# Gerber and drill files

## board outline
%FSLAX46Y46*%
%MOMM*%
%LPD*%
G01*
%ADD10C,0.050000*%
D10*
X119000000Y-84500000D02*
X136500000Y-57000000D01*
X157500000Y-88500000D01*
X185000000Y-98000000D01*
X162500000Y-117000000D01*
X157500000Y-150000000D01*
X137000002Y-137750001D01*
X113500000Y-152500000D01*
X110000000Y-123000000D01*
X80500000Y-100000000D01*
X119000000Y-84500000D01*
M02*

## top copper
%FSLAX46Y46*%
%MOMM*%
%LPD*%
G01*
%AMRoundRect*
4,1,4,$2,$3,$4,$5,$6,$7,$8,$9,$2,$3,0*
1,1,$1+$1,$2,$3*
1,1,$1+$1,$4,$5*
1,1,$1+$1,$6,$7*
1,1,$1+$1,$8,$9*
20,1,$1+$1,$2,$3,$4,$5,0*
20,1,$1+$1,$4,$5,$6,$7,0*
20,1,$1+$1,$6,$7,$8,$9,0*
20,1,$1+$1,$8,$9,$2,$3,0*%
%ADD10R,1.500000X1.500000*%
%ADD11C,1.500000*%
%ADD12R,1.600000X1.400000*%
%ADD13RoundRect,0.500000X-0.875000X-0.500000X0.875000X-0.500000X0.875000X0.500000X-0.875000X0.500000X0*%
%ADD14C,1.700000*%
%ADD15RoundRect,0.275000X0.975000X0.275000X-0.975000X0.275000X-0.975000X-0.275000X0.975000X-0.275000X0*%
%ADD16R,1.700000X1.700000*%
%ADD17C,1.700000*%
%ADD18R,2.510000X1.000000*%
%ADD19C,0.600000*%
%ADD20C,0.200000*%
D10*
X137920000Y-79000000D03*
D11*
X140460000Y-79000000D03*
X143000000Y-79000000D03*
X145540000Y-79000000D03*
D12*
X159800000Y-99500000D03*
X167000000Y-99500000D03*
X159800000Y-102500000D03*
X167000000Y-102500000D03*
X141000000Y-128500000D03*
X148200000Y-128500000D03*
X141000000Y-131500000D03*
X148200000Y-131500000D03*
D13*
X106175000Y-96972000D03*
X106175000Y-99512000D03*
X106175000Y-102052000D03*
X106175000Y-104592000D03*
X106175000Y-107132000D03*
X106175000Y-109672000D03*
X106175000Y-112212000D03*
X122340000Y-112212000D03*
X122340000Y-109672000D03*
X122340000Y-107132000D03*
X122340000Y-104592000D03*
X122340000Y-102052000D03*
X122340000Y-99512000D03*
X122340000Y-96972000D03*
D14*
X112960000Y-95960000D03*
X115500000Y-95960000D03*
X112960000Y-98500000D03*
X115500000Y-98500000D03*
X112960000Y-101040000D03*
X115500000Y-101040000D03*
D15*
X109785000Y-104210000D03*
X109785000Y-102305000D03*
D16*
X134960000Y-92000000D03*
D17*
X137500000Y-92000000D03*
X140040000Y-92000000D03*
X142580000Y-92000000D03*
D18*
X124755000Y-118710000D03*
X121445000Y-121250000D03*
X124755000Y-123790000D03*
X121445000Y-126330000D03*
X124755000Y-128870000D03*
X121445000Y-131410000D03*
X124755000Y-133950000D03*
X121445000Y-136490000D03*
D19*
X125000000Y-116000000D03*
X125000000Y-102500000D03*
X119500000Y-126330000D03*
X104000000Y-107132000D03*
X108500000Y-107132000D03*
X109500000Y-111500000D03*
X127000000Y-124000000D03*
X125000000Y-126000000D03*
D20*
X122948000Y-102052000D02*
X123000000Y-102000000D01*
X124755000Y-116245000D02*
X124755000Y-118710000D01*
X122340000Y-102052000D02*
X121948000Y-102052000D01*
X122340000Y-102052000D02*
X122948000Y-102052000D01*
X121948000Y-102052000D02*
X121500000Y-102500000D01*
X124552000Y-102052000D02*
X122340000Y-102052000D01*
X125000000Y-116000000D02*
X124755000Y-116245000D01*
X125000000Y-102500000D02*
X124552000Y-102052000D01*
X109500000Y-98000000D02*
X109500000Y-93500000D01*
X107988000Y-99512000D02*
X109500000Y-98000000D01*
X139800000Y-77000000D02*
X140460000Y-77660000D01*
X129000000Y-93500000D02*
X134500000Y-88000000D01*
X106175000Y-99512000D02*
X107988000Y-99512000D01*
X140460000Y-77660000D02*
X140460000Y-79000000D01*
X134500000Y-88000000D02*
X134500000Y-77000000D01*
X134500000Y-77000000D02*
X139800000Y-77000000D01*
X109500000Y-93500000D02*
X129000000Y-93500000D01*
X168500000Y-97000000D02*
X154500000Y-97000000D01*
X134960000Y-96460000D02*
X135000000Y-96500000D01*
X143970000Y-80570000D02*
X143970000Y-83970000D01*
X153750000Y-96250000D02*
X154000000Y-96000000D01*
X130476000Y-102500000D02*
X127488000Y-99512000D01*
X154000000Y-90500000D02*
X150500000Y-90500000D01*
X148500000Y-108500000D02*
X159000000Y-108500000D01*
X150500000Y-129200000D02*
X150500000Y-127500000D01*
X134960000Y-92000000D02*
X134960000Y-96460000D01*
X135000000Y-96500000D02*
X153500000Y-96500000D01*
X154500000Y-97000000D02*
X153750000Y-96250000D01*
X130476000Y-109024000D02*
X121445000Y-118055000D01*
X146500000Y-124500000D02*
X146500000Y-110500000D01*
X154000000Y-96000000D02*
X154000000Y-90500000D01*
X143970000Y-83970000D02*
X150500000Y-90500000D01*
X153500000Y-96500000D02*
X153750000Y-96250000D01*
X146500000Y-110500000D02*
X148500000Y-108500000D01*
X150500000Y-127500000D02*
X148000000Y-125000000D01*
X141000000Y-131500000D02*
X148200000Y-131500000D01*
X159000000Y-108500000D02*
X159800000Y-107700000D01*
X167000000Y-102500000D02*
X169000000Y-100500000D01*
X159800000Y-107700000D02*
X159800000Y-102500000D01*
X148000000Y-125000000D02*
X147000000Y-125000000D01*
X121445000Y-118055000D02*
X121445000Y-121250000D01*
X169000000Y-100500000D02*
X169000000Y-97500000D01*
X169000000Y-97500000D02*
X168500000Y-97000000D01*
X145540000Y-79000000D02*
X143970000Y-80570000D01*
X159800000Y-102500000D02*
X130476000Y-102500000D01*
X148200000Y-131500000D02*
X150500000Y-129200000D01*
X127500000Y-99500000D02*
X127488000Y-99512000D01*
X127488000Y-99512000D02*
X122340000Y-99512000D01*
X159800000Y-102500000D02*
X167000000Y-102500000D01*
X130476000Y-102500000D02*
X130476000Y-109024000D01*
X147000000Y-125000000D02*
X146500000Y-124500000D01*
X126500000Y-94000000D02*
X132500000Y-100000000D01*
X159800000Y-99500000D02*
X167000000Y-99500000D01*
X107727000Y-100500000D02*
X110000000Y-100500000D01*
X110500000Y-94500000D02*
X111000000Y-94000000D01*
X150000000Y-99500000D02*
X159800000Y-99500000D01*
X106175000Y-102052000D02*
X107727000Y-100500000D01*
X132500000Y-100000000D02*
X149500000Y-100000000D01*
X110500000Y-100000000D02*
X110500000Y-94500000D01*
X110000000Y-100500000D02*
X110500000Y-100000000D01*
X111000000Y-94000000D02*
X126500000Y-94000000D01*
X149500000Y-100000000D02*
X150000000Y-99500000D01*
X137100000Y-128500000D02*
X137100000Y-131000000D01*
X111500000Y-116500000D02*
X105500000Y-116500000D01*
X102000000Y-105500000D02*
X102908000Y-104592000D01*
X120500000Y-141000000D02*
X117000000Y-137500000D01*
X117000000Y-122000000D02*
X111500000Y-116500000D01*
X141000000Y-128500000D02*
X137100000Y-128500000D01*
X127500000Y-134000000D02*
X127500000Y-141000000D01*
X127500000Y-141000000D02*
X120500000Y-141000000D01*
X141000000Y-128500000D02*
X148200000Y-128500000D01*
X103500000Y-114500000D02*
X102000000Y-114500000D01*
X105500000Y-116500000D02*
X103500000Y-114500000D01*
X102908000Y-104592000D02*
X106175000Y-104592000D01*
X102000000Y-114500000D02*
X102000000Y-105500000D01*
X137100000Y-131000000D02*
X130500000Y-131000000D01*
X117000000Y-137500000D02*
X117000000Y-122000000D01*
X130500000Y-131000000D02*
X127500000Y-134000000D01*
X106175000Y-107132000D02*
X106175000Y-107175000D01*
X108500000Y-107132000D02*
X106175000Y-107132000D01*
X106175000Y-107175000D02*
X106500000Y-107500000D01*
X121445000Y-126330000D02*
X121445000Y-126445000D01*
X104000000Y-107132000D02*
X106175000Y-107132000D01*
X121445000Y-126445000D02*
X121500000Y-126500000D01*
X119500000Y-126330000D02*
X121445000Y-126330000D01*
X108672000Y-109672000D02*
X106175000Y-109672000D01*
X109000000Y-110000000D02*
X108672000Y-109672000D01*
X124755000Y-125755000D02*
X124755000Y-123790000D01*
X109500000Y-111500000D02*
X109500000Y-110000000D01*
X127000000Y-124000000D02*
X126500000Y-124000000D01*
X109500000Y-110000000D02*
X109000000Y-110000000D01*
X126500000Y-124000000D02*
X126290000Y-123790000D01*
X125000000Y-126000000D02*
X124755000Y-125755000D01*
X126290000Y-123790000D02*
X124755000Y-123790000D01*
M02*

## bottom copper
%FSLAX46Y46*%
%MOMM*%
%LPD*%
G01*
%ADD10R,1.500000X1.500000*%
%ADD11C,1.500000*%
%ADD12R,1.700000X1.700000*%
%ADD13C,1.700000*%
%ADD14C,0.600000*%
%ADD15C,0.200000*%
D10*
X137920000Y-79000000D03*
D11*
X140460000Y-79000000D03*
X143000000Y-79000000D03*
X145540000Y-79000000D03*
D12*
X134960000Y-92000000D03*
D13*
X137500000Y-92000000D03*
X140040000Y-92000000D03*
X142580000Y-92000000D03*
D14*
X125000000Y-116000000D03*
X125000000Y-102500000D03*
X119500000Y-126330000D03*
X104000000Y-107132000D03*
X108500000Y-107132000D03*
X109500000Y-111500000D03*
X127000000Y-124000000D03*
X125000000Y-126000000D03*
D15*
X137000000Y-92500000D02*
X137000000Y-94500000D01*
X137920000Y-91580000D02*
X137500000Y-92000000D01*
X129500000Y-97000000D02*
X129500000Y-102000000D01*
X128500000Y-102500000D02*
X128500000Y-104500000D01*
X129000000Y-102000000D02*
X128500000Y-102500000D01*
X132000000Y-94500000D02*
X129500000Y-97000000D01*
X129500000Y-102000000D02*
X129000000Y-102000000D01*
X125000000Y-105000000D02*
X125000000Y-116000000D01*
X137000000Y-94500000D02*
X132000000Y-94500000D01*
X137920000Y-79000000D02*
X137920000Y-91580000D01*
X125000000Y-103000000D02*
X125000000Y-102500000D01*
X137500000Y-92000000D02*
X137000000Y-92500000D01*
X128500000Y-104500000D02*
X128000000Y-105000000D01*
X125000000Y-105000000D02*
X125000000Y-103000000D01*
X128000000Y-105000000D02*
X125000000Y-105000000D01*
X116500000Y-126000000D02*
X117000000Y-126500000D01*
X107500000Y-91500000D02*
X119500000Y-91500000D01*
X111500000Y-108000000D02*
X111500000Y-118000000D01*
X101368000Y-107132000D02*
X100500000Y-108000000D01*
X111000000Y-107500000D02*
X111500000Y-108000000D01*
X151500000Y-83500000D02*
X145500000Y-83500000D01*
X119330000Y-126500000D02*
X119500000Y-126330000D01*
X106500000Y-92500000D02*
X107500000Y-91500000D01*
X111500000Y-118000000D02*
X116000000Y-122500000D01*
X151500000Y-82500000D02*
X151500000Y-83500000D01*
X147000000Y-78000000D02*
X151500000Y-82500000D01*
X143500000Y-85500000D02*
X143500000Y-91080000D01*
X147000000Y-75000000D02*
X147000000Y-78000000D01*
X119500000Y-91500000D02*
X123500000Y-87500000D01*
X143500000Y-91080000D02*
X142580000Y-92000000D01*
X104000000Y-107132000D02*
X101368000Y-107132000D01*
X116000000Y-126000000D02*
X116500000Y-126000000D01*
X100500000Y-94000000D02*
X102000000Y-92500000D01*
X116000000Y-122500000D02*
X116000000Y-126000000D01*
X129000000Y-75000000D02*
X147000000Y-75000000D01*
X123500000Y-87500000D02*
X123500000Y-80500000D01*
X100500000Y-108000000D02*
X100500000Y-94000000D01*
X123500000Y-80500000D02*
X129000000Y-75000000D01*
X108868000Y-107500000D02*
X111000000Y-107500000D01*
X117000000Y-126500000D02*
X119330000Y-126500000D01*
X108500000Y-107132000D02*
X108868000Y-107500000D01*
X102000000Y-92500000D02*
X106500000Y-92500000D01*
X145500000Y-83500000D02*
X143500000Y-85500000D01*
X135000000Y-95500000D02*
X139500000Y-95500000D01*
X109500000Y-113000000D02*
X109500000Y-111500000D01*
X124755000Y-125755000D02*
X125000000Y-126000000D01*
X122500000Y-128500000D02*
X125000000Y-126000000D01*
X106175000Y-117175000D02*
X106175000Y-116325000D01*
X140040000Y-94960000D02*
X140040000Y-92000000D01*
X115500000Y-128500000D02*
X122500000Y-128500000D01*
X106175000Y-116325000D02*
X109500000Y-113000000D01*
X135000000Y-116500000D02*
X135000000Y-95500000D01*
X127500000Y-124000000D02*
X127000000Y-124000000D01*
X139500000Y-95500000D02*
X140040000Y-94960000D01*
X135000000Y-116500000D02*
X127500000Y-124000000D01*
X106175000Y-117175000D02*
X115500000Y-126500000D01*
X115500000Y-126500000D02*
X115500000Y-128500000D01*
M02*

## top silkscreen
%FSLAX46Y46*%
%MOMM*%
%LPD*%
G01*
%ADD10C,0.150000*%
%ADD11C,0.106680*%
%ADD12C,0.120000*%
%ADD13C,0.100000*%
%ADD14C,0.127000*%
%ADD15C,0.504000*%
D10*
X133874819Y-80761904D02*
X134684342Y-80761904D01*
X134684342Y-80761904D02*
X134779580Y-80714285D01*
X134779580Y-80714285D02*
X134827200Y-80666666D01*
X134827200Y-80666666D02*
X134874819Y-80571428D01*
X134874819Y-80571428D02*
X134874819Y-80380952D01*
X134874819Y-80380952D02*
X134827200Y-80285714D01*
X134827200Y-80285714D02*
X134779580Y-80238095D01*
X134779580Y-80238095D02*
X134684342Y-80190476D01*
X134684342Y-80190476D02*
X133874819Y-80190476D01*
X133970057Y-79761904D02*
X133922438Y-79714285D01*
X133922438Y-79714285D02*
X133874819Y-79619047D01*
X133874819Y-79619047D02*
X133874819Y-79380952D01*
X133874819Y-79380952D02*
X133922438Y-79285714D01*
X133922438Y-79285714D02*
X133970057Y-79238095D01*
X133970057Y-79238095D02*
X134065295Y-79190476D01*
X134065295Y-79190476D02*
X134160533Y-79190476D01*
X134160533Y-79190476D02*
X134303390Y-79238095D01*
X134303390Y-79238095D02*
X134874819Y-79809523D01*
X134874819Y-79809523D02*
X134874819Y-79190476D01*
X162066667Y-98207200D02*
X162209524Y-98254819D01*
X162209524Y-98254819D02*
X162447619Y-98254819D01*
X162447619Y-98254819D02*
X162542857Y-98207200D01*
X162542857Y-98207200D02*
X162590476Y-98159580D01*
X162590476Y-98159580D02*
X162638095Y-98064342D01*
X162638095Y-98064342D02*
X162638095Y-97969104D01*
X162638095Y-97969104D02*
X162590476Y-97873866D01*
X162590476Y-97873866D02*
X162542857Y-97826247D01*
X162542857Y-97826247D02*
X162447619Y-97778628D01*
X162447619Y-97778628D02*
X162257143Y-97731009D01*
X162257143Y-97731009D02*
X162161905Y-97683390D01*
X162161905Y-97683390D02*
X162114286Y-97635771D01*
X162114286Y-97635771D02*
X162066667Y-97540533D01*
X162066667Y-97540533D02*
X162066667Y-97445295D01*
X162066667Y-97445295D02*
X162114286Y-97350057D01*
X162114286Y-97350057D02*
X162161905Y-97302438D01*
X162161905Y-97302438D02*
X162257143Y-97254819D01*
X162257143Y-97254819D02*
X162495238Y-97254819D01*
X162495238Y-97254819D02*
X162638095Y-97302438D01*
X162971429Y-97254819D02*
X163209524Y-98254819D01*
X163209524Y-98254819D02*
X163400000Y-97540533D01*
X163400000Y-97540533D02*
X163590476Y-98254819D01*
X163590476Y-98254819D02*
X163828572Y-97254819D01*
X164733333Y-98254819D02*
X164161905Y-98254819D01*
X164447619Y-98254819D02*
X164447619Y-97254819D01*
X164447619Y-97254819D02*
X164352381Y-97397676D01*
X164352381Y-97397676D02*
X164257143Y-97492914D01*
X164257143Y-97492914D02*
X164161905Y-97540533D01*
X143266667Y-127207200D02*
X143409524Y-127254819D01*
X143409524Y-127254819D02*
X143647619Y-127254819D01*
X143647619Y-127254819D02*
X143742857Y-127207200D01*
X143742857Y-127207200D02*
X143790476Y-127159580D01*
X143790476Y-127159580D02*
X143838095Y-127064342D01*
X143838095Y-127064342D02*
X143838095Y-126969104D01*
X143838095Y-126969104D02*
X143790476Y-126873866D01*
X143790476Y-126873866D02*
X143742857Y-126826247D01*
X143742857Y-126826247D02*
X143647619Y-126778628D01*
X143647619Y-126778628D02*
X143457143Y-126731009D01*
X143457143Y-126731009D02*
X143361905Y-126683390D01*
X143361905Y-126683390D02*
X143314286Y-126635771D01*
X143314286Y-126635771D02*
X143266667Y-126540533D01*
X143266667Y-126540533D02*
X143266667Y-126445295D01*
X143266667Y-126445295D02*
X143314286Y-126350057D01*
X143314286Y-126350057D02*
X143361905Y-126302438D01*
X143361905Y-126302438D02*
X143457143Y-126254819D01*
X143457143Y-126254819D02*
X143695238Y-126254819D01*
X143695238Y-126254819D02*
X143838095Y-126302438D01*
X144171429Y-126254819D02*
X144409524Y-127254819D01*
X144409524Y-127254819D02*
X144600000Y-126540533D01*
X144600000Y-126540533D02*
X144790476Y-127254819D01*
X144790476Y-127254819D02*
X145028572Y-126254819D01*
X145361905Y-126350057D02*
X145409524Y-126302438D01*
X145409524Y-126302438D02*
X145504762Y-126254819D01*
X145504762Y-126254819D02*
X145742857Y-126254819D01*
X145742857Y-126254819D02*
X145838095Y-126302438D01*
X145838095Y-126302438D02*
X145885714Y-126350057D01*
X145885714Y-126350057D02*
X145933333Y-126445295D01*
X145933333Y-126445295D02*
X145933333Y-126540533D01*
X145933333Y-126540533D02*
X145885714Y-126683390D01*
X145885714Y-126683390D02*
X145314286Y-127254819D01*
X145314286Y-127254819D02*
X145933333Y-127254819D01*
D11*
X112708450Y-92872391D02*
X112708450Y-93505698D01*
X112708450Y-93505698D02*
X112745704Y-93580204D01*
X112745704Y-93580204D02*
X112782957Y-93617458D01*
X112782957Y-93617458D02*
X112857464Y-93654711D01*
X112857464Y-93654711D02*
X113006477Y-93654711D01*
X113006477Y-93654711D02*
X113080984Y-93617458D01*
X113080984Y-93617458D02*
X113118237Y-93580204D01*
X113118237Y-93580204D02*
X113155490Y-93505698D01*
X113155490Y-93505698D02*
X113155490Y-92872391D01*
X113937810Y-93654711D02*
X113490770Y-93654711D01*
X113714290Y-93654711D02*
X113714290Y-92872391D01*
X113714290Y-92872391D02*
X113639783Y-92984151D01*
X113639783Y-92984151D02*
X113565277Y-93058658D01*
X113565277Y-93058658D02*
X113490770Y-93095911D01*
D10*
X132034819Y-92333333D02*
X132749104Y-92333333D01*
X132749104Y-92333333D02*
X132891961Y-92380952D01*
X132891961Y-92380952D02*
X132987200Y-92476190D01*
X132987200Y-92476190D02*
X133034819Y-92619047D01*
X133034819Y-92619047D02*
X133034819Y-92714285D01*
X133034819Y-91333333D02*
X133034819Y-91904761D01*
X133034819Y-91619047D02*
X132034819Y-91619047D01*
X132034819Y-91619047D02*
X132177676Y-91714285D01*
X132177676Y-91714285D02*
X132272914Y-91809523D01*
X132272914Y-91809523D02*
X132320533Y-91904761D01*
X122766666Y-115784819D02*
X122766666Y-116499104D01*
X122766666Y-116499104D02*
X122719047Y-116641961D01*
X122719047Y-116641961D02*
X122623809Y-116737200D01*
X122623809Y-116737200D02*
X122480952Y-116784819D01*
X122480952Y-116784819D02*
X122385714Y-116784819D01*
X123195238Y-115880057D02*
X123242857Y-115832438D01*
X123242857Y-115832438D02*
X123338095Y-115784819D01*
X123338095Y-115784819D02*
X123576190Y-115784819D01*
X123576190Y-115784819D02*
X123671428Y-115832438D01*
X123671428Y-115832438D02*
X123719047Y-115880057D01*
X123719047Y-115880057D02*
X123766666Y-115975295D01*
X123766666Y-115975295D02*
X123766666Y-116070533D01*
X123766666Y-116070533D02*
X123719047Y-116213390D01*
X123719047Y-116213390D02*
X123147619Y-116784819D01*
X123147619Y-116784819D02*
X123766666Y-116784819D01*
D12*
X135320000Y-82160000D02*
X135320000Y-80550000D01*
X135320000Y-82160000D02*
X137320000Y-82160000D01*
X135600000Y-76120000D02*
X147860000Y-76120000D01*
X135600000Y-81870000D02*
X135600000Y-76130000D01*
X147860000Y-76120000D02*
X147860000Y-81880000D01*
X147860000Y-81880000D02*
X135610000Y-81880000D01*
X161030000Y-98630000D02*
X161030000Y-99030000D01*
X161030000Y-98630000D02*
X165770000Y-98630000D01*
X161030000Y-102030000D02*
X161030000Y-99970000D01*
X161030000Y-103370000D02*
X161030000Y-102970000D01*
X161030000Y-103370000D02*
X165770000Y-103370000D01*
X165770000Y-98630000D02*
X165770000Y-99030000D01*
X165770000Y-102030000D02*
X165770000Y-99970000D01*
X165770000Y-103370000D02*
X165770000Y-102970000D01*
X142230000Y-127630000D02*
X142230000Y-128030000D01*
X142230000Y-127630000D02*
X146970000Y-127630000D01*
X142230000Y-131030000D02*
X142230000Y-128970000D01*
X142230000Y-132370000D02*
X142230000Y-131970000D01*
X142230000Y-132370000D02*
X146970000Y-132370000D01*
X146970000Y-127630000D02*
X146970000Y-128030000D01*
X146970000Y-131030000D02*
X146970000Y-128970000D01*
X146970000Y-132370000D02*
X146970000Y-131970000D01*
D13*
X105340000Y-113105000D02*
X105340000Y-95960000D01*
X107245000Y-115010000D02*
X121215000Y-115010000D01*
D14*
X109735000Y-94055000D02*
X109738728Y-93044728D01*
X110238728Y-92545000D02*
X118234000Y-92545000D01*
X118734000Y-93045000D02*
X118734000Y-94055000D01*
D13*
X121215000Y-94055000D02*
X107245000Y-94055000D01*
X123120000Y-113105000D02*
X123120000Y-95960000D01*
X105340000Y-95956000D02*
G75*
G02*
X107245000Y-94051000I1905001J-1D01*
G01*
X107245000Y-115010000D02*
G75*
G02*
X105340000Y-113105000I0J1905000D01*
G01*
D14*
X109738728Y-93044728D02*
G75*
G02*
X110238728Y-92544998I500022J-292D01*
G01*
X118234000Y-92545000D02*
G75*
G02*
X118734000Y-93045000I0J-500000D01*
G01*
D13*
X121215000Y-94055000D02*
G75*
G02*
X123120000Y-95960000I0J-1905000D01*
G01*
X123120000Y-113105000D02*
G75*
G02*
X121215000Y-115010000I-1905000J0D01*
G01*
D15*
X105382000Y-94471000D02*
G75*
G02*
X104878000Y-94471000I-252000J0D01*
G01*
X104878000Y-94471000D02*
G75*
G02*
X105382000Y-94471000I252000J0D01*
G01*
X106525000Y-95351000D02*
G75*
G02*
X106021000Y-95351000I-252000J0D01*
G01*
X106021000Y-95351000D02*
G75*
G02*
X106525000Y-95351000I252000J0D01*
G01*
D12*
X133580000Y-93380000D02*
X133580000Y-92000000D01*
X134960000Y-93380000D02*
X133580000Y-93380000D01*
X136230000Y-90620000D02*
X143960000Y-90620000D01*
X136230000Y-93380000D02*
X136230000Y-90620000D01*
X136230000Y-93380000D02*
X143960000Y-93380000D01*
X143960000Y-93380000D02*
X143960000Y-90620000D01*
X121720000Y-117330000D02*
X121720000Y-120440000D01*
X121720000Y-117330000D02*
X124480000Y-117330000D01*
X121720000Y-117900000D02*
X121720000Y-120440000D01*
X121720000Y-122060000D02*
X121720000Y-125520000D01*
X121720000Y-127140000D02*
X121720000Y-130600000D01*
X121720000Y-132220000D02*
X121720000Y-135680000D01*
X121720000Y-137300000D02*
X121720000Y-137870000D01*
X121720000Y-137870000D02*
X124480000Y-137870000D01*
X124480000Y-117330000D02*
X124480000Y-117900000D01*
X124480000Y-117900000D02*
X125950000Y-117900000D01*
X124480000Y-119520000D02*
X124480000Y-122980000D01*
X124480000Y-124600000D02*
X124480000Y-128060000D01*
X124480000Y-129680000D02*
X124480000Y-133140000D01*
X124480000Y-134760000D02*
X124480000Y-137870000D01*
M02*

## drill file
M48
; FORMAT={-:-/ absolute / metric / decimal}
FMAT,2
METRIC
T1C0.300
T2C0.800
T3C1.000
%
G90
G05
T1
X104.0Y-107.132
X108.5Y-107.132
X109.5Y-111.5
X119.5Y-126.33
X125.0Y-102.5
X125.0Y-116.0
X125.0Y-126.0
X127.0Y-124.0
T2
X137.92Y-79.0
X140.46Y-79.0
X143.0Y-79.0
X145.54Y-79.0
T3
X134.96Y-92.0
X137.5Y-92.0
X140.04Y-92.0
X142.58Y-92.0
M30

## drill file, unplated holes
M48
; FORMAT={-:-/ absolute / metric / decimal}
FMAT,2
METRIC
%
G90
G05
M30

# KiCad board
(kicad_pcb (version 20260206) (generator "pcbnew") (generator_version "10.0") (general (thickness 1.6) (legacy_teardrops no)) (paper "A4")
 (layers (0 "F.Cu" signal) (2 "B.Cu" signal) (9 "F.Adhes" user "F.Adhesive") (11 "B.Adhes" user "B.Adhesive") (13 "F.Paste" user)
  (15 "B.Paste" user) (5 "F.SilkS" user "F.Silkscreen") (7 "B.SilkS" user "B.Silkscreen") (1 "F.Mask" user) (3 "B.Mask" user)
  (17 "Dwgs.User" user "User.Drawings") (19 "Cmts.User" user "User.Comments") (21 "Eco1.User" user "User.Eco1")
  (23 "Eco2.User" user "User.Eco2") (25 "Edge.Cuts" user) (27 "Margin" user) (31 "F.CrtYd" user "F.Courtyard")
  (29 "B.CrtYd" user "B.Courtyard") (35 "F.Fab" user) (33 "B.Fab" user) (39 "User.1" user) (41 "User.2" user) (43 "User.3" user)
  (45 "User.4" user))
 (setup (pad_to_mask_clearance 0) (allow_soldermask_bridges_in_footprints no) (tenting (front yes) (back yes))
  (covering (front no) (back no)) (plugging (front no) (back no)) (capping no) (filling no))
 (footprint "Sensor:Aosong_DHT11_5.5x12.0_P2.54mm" (layer "F.Cu") (at 137.92 79 90)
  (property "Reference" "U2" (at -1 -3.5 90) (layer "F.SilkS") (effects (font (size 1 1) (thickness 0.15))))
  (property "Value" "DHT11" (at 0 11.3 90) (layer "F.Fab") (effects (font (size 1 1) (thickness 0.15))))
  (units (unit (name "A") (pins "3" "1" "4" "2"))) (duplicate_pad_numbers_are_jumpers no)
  (fp_line (start -3.16 -2.6) (end -1.55 -2.6) (stroke (width 0.12) (type solid)) (layer "F.SilkS"))
  (fp_line (start -3.16 -2.6) (end -3.16 -0.6) (stroke (width 0.12) (type solid)) (layer "F.SilkS"))
  (fp_line (start 2.88 -2.32) (end 2.88 9.94) (stroke (width 0.12) (type solid)) (layer "F.SilkS"))
  (fp_line (start -2.87 -2.32) (end 2.87 -2.32) (stroke (width 0.12) (type solid)) (layer "F.SilkS"))
  (fp_line (start 2.88 9.94) (end -2.88 9.94) (stroke (width 0.12) (type solid)) (layer "F.SilkS"))
  (fp_line (start -2.88 9.94) (end -2.88 -2.31) (stroke (width 0.12) (type solid)) (layer "F.SilkS"))
  (pad "1" thru_hole rect (at 0 0 90) (size 1.5 1.5) (drill 0.8) (layers "*.Cu" "*.Mask") (remove_unused_layers no) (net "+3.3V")
   (padstack (mode custom) (layer "B.Cu" (shape rect) (size 1.5 1.5))))
  (pad "2" thru_hole circle (at 0 2.54 90) (size 1.5 1.5) (drill 0.8) (layers "*.Cu" "*.Mask") (remove_unused_layers no) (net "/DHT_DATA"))
  (pad "3" thru_hole circle (at 0 5.08 90) (size 1.5 1.5) (drill 0.8) (layers "*.Cu" "*.Mask") (remove_unused_layers no)
   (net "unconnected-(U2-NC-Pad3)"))
  (pad "4" thru_hole circle (at 0 7.62 90) (size 1.5 1.5) (drill 0.8) (layers "*.Cu" "*.Mask") (remove_unused_layers no) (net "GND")))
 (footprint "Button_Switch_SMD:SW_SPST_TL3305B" (layer "F.Cu") (at 163.4 101)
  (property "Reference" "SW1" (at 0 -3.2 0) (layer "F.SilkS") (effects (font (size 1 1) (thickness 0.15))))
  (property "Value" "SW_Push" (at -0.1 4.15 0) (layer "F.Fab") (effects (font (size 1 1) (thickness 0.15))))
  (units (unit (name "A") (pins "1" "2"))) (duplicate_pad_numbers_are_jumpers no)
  (fp_line (start -2.37 -2.37) (end -2.37 -1.97) (stroke (width 0.12) (type solid)) (layer "F.SilkS"))
  (fp_line (start -2.37 -2.37) (end 2.37 -2.37) (stroke (width 0.12) (type solid)) (layer "F.SilkS"))
  (fp_line (start -2.37 1.03) (end -2.37 -1.03) (stroke (width 0.12) (type solid)) (layer "F.SilkS"))
  (fp_line (start -2.37 2.37) (end -2.37 1.97) (stroke (width 0.12) (type solid)) (layer "F.SilkS"))
  (fp_line (start -2.37 2.37) (end 2.37 2.37) (stroke (width 0.12) (type solid)) (layer "F.SilkS"))
  (fp_line (start 2.37 -2.37) (end 2.37 -1.97) (stroke (width 0.12) (type solid)) (layer "F.SilkS"))
  (fp_line (start 2.37 1.03) (end 2.37 -1.03) (stroke (width 0.12) (type solid)) (layer "F.SilkS"))
  (fp_line (start 2.37 2.37) (end 2.37 1.97) (stroke (width 0.12) (type solid)) (layer "F.SilkS"))
  (pad "1" smd rect (at -3.6 -1.5) (size 1.6 1.4) (layers "F.Cu" "F.Mask" "F.Paste") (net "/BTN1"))
  (pad "1" smd rect (at 3.6 -1.5) (size 1.6 1.4) (layers "F.Cu" "F.Mask" "F.Paste") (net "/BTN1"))
  (pad "2" smd rect (at -3.6 1.5) (size 1.6 1.4) (layers "F.Cu" "F.Mask" "F.Paste") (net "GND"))
  (pad "2" smd rect (at 3.6 1.5) (size 1.6 1.4) (layers "F.Cu" "F.Mask" "F.Paste") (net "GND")))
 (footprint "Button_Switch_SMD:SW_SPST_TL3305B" (layer "F.Cu") (at 144.6 130)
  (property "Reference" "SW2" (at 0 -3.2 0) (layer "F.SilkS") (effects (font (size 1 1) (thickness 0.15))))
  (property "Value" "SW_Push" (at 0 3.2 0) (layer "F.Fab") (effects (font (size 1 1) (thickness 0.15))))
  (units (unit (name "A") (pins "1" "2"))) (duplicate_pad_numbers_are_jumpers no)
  (fp_line (start -2.37 -2.37) (end -2.37 -1.97) (stroke (width 0.12) (type solid)) (layer "F.SilkS"))
  (fp_line (start -2.37 -2.37) (end 2.37 -2.37) (stroke (width 0.12) (type solid)) (layer "F.SilkS"))
  (fp_line (start -2.37 1.03) (end -2.37 -1.03) (stroke (width 0.12) (type solid)) (layer "F.SilkS"))
  (fp_line (start -2.37 2.37) (end -2.37 1.97) (stroke (width 0.12) (type solid)) (layer "F.SilkS"))
  (fp_line (start -2.37 2.37) (end 2.37 2.37) (stroke (width 0.12) (type solid)) (layer "F.SilkS"))
  (fp_line (start 2.37 -2.37) (end 2.37 -1.97) (stroke (width 0.12) (type solid)) (layer "F.SilkS"))
  (fp_line (start 2.37 1.03) (end 2.37 -1.03) (stroke (width 0.12) (type solid)) (layer "F.SilkS"))
  (fp_line (start 2.37 2.37) (end 2.37 1.97) (stroke (width 0.12) (type solid)) (layer "F.SilkS"))
  (pad "1" smd rect (at -3.6 -1.5) (size 1.6 1.4) (layers "F.Cu" "F.Mask" "F.Paste") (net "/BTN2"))
  (pad "1" smd rect (at 3.6 -1.5) (size 1.6 1.4) (layers "F.Cu" "F.Mask" "F.Paste") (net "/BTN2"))
  (pad "2" smd rect (at -3.6 1.5) (size 1.6 1.4) (layers "F.Cu" "F.Mask" "F.Paste") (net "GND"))
  (pad "2" smd rect (at 3.6 1.5) (size 1.6 1.4) (layers "F.Cu" "F.Mask" "F.Paste") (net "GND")))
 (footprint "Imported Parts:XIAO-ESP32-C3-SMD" (layer "F.Cu") (at 105.34 115.092)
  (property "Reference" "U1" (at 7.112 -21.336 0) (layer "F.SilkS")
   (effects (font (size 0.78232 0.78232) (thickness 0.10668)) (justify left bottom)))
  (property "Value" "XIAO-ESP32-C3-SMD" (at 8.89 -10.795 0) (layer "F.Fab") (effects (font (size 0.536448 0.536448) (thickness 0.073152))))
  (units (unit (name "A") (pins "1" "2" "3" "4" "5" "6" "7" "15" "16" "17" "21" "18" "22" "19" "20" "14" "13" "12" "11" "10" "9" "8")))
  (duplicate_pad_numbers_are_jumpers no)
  (fp_line (start 0 -1.987) (end 0 -19.132) (stroke (width 0.1) (type solid)) (layer "F.SilkS"))
  (fp_line (start 1.905 -0.082) (end 15.875 -0.082) (stroke (width 0.1) (type solid)) (layer "F.SilkS"))
  (fp_line (start 4.395 -21.037) (end 4.398728 -22.047272) (stroke (width 0.127) (type solid)) (layer "F.SilkS"))
  (fp_line (start 4.898728 -22.547) (end 12.894 -22.547) (stroke (width 0.127) (type solid)) (layer "F.SilkS"))
  (fp_line (start 13.394 -22.047) (end 13.394 -21.037) (stroke (width 0.127) (type solid)) (layer "F.SilkS"))
  (fp_line (start 15.875 -21.037) (end 1.905 -21.037) (stroke (width 0.1) (type solid)) (layer "F.SilkS"))
  (fp_line (start 17.78 -1.987) (end 17.78 -19.132) (stroke (width 0.1) (type solid)) (layer "F.SilkS"))
  (fp_arc (start 0 -19.136) (mid 0.557962 -20.483038) (end 1.905 -21.041) (stroke (width 0.1) (type solid)) (layer "F.SilkS"))
  (fp_arc (start 1.905 -0.082) (mid 0.557962 -0.639962) (end 0 -1.987) (stroke (width 0.1) (type solid)) (layer "F.SilkS"))
  (fp_arc (start 4.398728 -22.047272) (mid 4.545272 -22.40064) (end 4.898728 -22.547) (stroke (width 0.127) (type default))
   (layer "F.SilkS"))
  (fp_arc (start 12.894 -22.547) (mid 13.247553 -22.400553) (end 13.394 -22.047) (stroke (width 0.127) (type default)) (layer "F.SilkS"))
  (fp_arc (start 15.875 -21.037) (mid 17.222038 -20.479038) (end 17.78 -19.132) (stroke (width 0.1) (type solid)) (layer "F.SilkS"))
  (fp_arc (start 17.78 -1.987) (mid 17.222038 -0.639962) (end 15.875 -0.082) (stroke (width 0.1) (type solid)) (layer "F.SilkS"))
  (fp_circle (center -0.21 -20.621) (end -0.21 -20.875) (stroke (width 0.5) (type solid)) (fill yes) (layer "F.SilkS"))
  (fp_circle (center 0.933 -19.741) (end 0.933 -19.995) (stroke (width 0.5) (type solid)) (fill yes) (layer "F.SilkS"))
  (pad "1" smd roundrect (at 0.835 -18.12) (size 2.75 2) (layers "F.Cu" "F.Mask" "F.Paste") (roundrect_rratio 0.25)
   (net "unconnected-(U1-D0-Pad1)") (solder_mask_margin 0.0508) (thermal_bridge_angle 45))
  (pad "2" smd roundrect (at 0.835 -15.58) (size 2.75 2) (layers "F.Cu" "F.Mask" "F.Paste") (roundrect_rratio 0.25) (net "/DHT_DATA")
   (solder_mask_margin 0.0508) (thermal_bridge_angle 45))
  (pad "3" smd roundrect (at 0.835 -13.04) (size 2.75 2) (layers "F.Cu" "F.Mask" "F.Paste") (roundrect_rratio 0.25) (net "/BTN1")
   (solder_mask_margin 0.0508) (thermal_bridge_angle 45))
  (pad "4" smd roundrect (at 0.835 -10.5) (size 2.75 2) (layers "F.Cu" "F.Mask" "F.Paste") (roundrect_rratio 0.25) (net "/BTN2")
   (solder_mask_margin 0.0508) (thermal_bridge_angle 45))
  (pad "5" smd roundrect (at 0.835 -7.96) (size 2.75 2) (layers "F.Cu" "F.Mask" "F.Paste") (roundrect_rratio 0.25) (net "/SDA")
   (solder_mask_margin 0.0508) (thermal_bridge_angle 45)
   (padstack (mode custom) (layer "B.Cu" (shape roundrect) (size 2.75 2) (roundrect_rratio 0.25))))
  (pad "6" smd roundrect (at 0.835 -5.42) (size 2.75 2) (layers "F.Cu" "F.Mask" "F.Paste") (roundrect_rratio 0.25) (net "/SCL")
   (solder_mask_margin 0.0508) (thermal_bridge_angle 45))
  (pad "7" smd roundrect (at 0.835 -2.88) (size 2.75 2) (layers "F.Cu" "F.Mask" "F.Paste") (roundrect_rratio 0.25)
   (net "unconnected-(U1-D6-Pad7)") (solder_mask_margin 0.0508) (thermal_bridge_angle 45))
  (pad "8" smd roundrect (at 17 -2.88) (size 2.75 2) (layers "F.Cu" "F.Mask" "F.Paste") (roundrect_rratio 0.25)
   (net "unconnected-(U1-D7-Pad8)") (solder_mask_margin 0.0508) (thermal_bridge_angle 45))
  (pad "9" smd roundrect (at 17 -5.42) (size 2.75 2) (layers "F.Cu" "F.Mask" "F.Paste") (roundrect_rratio 0.25)
   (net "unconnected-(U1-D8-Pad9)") (solder_mask_margin 0.0508) (thermal_bridge_angle 45))
  (pad "10" smd roundrect (at 17 -7.96) (size 2.75 2) (layers "F.Cu" "F.Mask" "F.Paste") (roundrect_rratio 0.25)
   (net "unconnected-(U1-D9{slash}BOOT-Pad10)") (solder_mask_margin 0.0508) (thermal_bridge_angle 45))
  (pad "11" smd roundrect (at 17 -10.5) (size 2.75 2) (layers "F.Cu" "F.Mask" "F.Paste") (roundrect_rratio 0.25)
   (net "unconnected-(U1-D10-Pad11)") (solder_mask_margin 0.0508) (thermal_bridge_angle 45))
  (pad "12" smd roundrect (at 17 -13.04) (size 2.75 2) (layers "F.Cu" "F.Mask" "F.Paste") (roundrect_rratio 0.25) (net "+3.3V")
   (solder_mask_margin 0.0508) (thermal_bridge_angle 45)
   (padstack (mode custom) (layer "B.Cu" (shape roundrect) (size 2.75 2) (roundrect_rratio 0.25))))
  (pad "13" smd roundrect (at 17 -15.58) (size 2.75 2) (layers "F.Cu" "F.Mask" "F.Paste") (roundrect_rratio 0.25) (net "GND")
   (solder_mask_margin 0.0508) (thermal_bridge_angle 45))
  (pad "14" smd roundrect (at 17 -18.12) (size 2.75 2) (layers "F.Cu" "F.Mask" "F.Paste") (roundrect_rratio 0.25) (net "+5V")
   (solder_mask_margin 0.0508) (thermal_bridge_angle 45))
  (pad "15" smd circle (at 7.62 -19.132) (size 1.7 1.7) (layers "F.Cu" "F.Mask" "F.Paste") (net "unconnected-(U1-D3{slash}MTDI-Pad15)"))
  (pad "16" smd circle (at 10.16 -19.132) (size 1.7 1.7) (layers "F.Cu" "F.Mask" "F.Paste") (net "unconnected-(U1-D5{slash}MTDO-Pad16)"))
  (pad "17" smd circle (at 7.62 -16.592) (size 1.7 1.7) (layers "F.Cu" "F.Mask" "F.Paste") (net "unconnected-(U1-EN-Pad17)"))
  (pad "18" smd circle (at 10.16 -16.592) (size 1.7 1.7) (layers "F.Cu" "F.Mask" "F.Paste") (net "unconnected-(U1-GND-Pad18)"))
  (pad "19" smd circle (at 7.62 -14.052) (size 1.7 1.7) (layers "F.Cu" "F.Mask" "F.Paste") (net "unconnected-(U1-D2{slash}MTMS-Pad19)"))
  (pad "20" smd circle (at 10.16 -14.052) (size 1.7 1.7) (layers "F.Cu" "F.Mask" "F.Paste") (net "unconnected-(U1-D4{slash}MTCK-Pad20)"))
  (pad "21" smd roundrect (at 4.445 -10.882 180) (size 2.5 1.1) (layers "F.Cu" "F.Mask" "F.Paste") (roundrect_rratio 0.25)
   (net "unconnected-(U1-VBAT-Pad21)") (thermal_bridge_angle 45))
  (pad "22" smd roundrect (at 4.445 -12.787 180) (size 2.5 1.1) (layers "F.Cu" "F.Mask" "F.Paste") (roundrect_rratio 0.25)
   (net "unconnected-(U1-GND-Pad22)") (thermal_bridge_angle 45)))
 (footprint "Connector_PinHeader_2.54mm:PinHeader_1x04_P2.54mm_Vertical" (layer "F.Cu") (at 134.96 92 90)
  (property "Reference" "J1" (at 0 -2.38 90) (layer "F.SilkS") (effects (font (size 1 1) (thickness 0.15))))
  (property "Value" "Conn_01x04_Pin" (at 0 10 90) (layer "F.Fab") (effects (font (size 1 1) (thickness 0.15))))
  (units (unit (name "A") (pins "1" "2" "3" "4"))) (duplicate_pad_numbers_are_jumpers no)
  (fp_line (start -1.38 -1.38) (end 0 -1.38) (stroke (width 0.12) (type solid)) (layer "F.SilkS"))
  (fp_line (start -1.38 0) (end -1.38 -1.38) (stroke (width 0.12) (type solid)) (layer "F.SilkS"))
  (fp_line (start 1.38 1.27) (end 1.38 9) (stroke (width 0.12) (type solid)) (layer "F.SilkS"))
  (fp_line (start -1.38 1.27) (end 1.38 1.27) (stroke (width 0.12) (type solid)) (layer "F.SilkS"))
  (fp_line (start -1.38 1.27) (end -1.38 9) (stroke (width 0.12) (type solid)) (layer "F.SilkS"))
  (fp_line (start -1.38 9) (end 1.38 9) (stroke (width 0.12) (type solid)) (layer "F.SilkS"))
  (pad "1" thru_hole rect (at 0 0 90) (size 1.7 1.7) (drill 1) (layers "*.Cu" "*.Mask") (remove_unused_layers no) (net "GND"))
  (pad "2" thru_hole circle (at 0 2.54 90) (size 1.7 1.7) (drill 1) (layers "*.Cu" "*.Mask") (remove_unused_layers no) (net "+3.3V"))
  (pad "3" thru_hole circle (at 0 5.08 90) (size 1.7 1.7) (drill 1) (layers "*.Cu" "*.Mask") (remove_unused_layers no) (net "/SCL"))
  (pad "4" thru_hole circle (at 0 7.62 90) (size 1.7 1.7) (drill 1) (layers "*.Cu" "*.Mask") (remove_unused_layers no) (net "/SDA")))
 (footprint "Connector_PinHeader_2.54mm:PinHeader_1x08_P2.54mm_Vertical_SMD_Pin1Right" (layer "F.Cu") (at 123.1 127.6)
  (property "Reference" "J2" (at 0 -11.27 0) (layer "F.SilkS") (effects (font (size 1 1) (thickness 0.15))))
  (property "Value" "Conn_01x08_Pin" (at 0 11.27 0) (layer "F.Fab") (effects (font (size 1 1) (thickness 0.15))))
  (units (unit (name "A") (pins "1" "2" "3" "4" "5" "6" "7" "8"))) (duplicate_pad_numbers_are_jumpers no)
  (fp_line (start -1.38 -10.27) (end -1.38 -7.16) (stroke (width 0.12) (type solid)) (layer "F.SilkS"))
  (fp_line (start -1.38 -10.27) (end 1.38 -10.27) (stroke (width 0.12) (type solid)) (layer "F.SilkS"))
  (fp_line (start -1.38 -9.7) (end -1.38 -7.16) (stroke (width 0.12) (type solid)) (layer "F.SilkS"))
  (fp_line (start -1.38 -5.54) (end -1.38 -2.08) (stroke (width 0.12) (type solid)) (layer "F.SilkS"))
  (fp_line (start -1.38 -0.46) (end -1.38 3) (stroke (width 0.12) (type solid)) (layer "F.SilkS"))
  (fp_line (start -1.38 4.62) (end -1.38 8.08) (stroke (width 0.12) (type solid)) (layer "F.SilkS"))
  (fp_line (start -1.38 9.7) (end -1.38 10.27) (stroke (width 0.12) (type solid)) (layer "F.SilkS"))
  (fp_line (start -1.38 10.27) (end 1.38 10.27) (stroke (width 0.12) (type solid)) (layer "F.SilkS"))
  (fp_line (start 1.38 -10.27) (end 1.38 -9.7) (stroke (width 0.12) (type solid)) (layer "F.SilkS"))
  (fp_line (start 1.38 -9.7) (end 2.85 -9.7) (stroke (width 0.12) (type solid)) (layer "F.SilkS"))
  (fp_line (start 1.38 -8.08) (end 1.38 -4.62) (stroke (width 0.12) (type solid)) (layer "F.SilkS"))
  (fp_line (start 1.38 -3) (end 1.38 0.46) (stroke (width 0.12) (type solid)) (layer "F.SilkS"))
  (fp_line (start 1.38 2.08) (end 1.38 5.54) (stroke (width 0.12) (type solid)) (layer "F.SilkS"))
  (fp_line (start 1.38 7.16) (end 1.38 10.27) (stroke (width 0.12) (type solid)) (layer "F.SilkS"))
  (pad "1" smd rect (at 1.655 -8.89) (size 2.51 1) (layers "F.Cu" "F.Mask" "F.Paste") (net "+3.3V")
   (padstack (mode custom) (layer "B.Cu" (shape rect) (size 2.51 1))))
  (pad "2" smd rect (at -1.655 -6.35) (size 2.51 1) (layers "F.Cu" "F.Mask" "F.Paste") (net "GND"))
  (pad "3" smd rect (at 1.655 -3.81) (size 2.51 1) (layers "F.Cu" "F.Mask" "F.Paste") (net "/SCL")
   (padstack (mode custom) (layer "B.Cu" (shape rect) (size 2.51 1))))
  (pad "4" smd rect (at -1.655 -1.27) (size 2.51 1) (layers "F.Cu" "F.Mask" "F.Paste") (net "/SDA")
   (padstack (mode custom) (layer "B.Cu" (shape rect) (size 2.51 1))))
  (pad "5" smd rect (at 1.655 1.27) (size 2.51 1) (layers "F.Cu" "F.Mask" "F.Paste") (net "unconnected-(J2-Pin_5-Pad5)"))
  (pad "6" smd rect (at -1.655 3.81) (size 2.51 1) (layers "F.Cu" "F.Mask" "F.Paste") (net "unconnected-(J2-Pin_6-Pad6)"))
  (pad "7" smd rect (at 1.655 6.35) (size 2.51 1) (layers "F.Cu" "F.Mask" "F.Paste") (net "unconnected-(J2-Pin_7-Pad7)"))
  (pad "8" smd rect (at -1.655 8.89) (size 2.51 1) (layers "F.Cu" "F.Mask" "F.Paste") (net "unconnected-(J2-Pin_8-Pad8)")))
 (gr_poly
  (pts (xy 119 84.5) (xy 136.5 57) (xy 157.5 88.5) (xy 185 98) (xy 162.5 117) (xy 157.5 150) (xy 137.000002 137.750001) (xy 113.5 152.5)
   (xy 110 123) (xy 80.5 100))
  (stroke (width 0.05) (type solid)) (fill no) (layer "Edge.Cuts"))
 (segment (start 122.948 102.052) (end 123 102) (width 0.2) (layer "F.Cu") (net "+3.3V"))
 (segment (start 124.755 116.245) (end 124.755 118.71) (width 0.2) (layer "F.Cu") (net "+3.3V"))
 (segment (start 122.34 102.052) (end 121.948 102.052) (width 0.2) (layer "F.Cu") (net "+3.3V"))
 (segment (start 122.34 102.052) (end 122.948 102.052) (width 0.2) (layer "F.Cu") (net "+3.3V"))
 (segment (start 121.948 102.052) (end 121.5 102.5) (width 0.2) (layer "F.Cu") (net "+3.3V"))
 (segment (start 124.552 102.052) (end 122.34 102.052) (width 0.2) (layer "F.Cu") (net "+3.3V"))
 (segment (start 125 116) (end 124.755 116.245) (width 0.2) (layer "F.Cu") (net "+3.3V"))
 (segment (start 125 102.5) (end 124.552 102.052) (width 0.2) (layer "F.Cu") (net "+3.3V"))
 (via (at 125 116) (size 0.6) (drill 0.3) (layers "F.Cu" "B.Cu") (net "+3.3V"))
 (via (at 125 102.5) (size 0.6) (drill 0.3) (layers "F.Cu" "B.Cu") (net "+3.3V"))
 (segment (start 137 92.5) (end 137 94.5) (width 0.2) (layer "B.Cu") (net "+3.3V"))
 (segment (start 137.92 91.58) (end 137.5 92) (width 0.2) (layer "B.Cu") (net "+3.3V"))
 (segment (start 129.5 97) (end 129.5 102) (width 0.2) (layer "B.Cu") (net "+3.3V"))
 (segment (start 128.5 102.5) (end 128.5 104.5) (width 0.2) (layer "B.Cu") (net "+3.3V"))
 (segment (start 129 102) (end 128.5 102.5) (width 0.2) (layer "B.Cu") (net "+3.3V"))
 (segment (start 132 94.5) (end 129.5 97) (width 0.2) (layer "B.Cu") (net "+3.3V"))
 (segment (start 129.5 102) (end 129 102) (width 0.2) (layer "B.Cu") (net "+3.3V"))
 (segment (start 125 105) (end 125 116) (width 0.2) (layer "B.Cu") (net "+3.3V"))
 (segment (start 137 94.5) (end 132 94.5) (width 0.2) (layer "B.Cu") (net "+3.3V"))
 (segment (start 137.92 79) (end 137.92 91.58) (width 0.2) (layer "B.Cu") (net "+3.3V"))
 (segment (start 125 103) (end 125 102.5) (width 0.2) (layer "B.Cu") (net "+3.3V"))
 (segment (start 137.5 92) (end 137 92.5) (width 0.2) (layer "B.Cu") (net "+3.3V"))
 (segment (start 128.5 104.5) (end 128 105) (width 0.2) (layer "B.Cu") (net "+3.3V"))
 (segment (start 125 105) (end 125 103) (width 0.2) (layer "B.Cu") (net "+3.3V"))
 (segment (start 128 105) (end 125 105) (width 0.2) (layer "B.Cu") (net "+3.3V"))
 (segment (start 109.5 98) (end 109.5 93.5) (width 0.2) (layer "F.Cu") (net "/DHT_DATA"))
 (segment (start 107.988 99.512) (end 109.5 98) (width 0.2) (layer "F.Cu") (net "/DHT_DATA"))
 (segment (start 139.8 77) (end 140.46 77.66) (width 0.2) (layer "F.Cu") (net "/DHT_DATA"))
 (segment (start 129 93.5) (end 134.5 88) (width 0.2) (layer "F.Cu") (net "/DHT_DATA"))
 (segment (start 106.175 99.512) (end 107.988 99.512) (width 0.2) (layer "F.Cu") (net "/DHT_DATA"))
 (segment (start 140.46 77.66) (end 140.46 79) (width 0.2) (layer "F.Cu") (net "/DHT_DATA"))
 (segment (start 134.5 88) (end 134.5 77) (width 0.2) (layer "F.Cu") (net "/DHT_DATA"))
 (segment (start 134.5 77) (end 139.8 77) (width 0.2) (layer "F.Cu") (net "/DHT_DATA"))
 (segment (start 109.5 93.5) (end 129 93.5) (width 0.2) (layer "F.Cu") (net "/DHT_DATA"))
 (segment (start 168.5 97) (end 154.5 97) (width 0.2) (layer "F.Cu") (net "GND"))
 (segment (start 134.96 96.46) (end 135 96.5) (width 0.2) (layer "F.Cu") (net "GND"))
 (segment (start 143.97 80.57) (end 143.97 83.97) (width 0.2) (layer "F.Cu") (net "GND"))
 (segment (start 153.75 96.25) (end 154 96) (width 0.2) (layer "F.Cu") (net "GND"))
 (segment (start 130.476 102.5) (end 127.488 99.512) (width 0.2) (layer "F.Cu") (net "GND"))
 (segment (start 154 90.5) (end 150.5 90.5) (width 0.2) (layer "F.Cu") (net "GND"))
 (segment (start 148.5 108.5) (end 159 108.5) (width 0.2) (layer "F.Cu") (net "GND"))
 (segment (start 150.5 129.2) (end 150.5 127.5) (width 0.2) (layer "F.Cu") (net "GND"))
 (segment (start 134.96 92) (end 134.96 96.46) (width 0.2) (layer "F.Cu") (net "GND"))
 (segment (start 135 96.5) (end 153.5 96.5) (width 0.2) (layer "F.Cu") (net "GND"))
 (segment (start 154.5 97) (end 153.75 96.25) (width 0.2) (layer "F.Cu") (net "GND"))
 (segment (start 130.476 109.024) (end 121.445 118.055) (width 0.2) (layer "F.Cu") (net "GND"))
 (segment (start 146.5 124.5) (end 146.5 110.5) (width 0.2) (layer "F.Cu") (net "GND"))
 (segment (start 154 96) (end 154 90.5) (width 0.2) (layer "F.Cu") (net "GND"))
 (segment (start 143.97 83.97) (end 150.5 90.5) (width 0.2) (layer "F.Cu") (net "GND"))
 (segment (start 153.5 96.5) (end 153.75 96.25) (width 0.2) (layer "F.Cu") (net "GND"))
 (segment (start 146.5 110.5) (end 148.5 108.5) (width 0.2) (layer "F.Cu") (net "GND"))
 (segment (start 150.5 127.5) (end 148 125) (width 0.2) (layer "F.Cu") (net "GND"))
 (segment (start 141 131.5) (end 148.2 131.5) (width 0.2) (layer "F.Cu") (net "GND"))
 (segment (start 159 108.5) (end 159.8 107.7) (width 0.2) (layer "F.Cu") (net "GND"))
 (segment (start 167 102.5) (end 169 100.5) (width 0.2) (layer "F.Cu") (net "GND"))
 (segment (start 159.8 107.7) (end 159.8 102.5) (width 0.2) (layer "F.Cu") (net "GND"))
 (segment (start 148 125) (end 147 125) (width 0.2) (layer "F.Cu") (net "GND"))
 (segment (start 121.445 118.055) (end 121.445 121.25) (width 0.2) (layer "F.Cu") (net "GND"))
 (segment (start 169 100.5) (end 169 97.5) (width 0.2) (layer "F.Cu") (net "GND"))
 (segment (start 169 97.5) (end 168.5 97) (width 0.2) (layer "F.Cu") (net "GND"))
 (segment (start 145.54 79) (end 143.97 80.57) (width 0.2) (layer "F.Cu") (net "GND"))
 (segment (start 159.8 102.5) (end 130.476 102.5) (width 0.2) (layer "F.Cu") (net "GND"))
 (segment (start 148.2 131.5) (end 150.5 129.2) (width 0.2) (layer "F.Cu") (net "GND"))
 (segment (start 127.5 99.5) (end 127.488 99.512) (width 0.2) (layer "F.Cu") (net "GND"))
 (segment (start 127.488 99.512) (end 122.34 99.512) (width 0.2) (layer "F.Cu") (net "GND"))
 (segment (start 159.8 102.5) (end 167 102.5) (width 0.2) (layer "F.Cu") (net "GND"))
 (segment (start 130.476 102.5) (end 130.476 109.024) (width 0.2) (layer "F.Cu") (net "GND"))
 (segment (start 147 125) (end 146.5 124.5) (width 0.2) (layer "F.Cu") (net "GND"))
 (segment (start 126.5 94) (end 132.5 100) (width 0.2) (layer "F.Cu") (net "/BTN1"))
 (segment (start 159.8 99.5) (end 167 99.5) (width 0.2) (layer "F.Cu") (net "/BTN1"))
 (segment (start 107.727 100.5) (end 110 100.5) (width 0.2) (layer "F.Cu") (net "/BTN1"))
 (segment (start 110.5 94.5) (end 111 94) (width 0.2) (layer "F.Cu") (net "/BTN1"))
 (segment (start 150 99.5) (end 159.8 99.5) (width 0.2) (layer "F.Cu") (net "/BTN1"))
 (segment (start 106.175 102.052) (end 107.727 100.5) (width 0.2) (layer "F.Cu") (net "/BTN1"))
 (segment (start 132.5 100) (end 149.5 100) (width 0.2) (layer "F.Cu") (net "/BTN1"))
 (segment (start 110.5 100) (end 110.5 94.5) (width 0.2) (layer "F.Cu") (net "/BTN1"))
 (segment (start 110 100.5) (end 110.5 100) (width 0.2) (layer "F.Cu") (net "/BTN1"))
 (segment (start 111 94) (end 126.5 94) (width 0.2) (layer "F.Cu") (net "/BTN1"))
 (segment (start 149.5 100) (end 150 99.5) (width 0.2) (layer "F.Cu") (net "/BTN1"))
 (segment (start 137.1 128.5) (end 137.1 131) (width 0.2) (layer "F.Cu") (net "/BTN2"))
 (segment (start 111.5 116.5) (end 105.5 116.5) (width 0.2) (layer "F.Cu") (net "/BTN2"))
 (segment (start 102 105.5) (end 102.908 104.592) (width 0.2) (layer "F.Cu") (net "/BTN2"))
 (segment (start 120.5 141) (end 117 137.5) (width 0.2) (layer "F.Cu") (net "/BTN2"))
 (segment (start 117 122) (end 111.5 116.5) (width 0.2) (layer "F.Cu") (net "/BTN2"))
 (segment (start 141 128.5) (end 137.1 128.5) (width 0.2) (layer "F.Cu") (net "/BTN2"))
 (segment (start 127.5 134) (end 127.5 141) (width 0.2) (layer "F.Cu") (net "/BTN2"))
 (segment (start 127.5 141) (end 120.5 141) (width 0.2) (layer "F.Cu") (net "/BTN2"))
 (segment (start 141 128.5) (end 148.2 128.5) (width 0.2) (layer "F.Cu") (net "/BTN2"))
 (segment (start 103.5 114.5) (end 102 114.5) (width 0.2) (layer "F.Cu") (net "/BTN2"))
 (segment (start 105.5 116.5) (end 103.5 114.5) (width 0.2) (layer "F.Cu") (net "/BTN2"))
 (segment (start 102.908 104.592) (end 106.175 104.592) (width 0.2) (layer "F.Cu") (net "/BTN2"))
 (segment (start 102 114.5) (end 102 105.5) (width 0.2) (layer "F.Cu") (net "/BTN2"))
 (segment (start 137.1 131) (end 130.5 131) (width 0.2) (layer "F.Cu") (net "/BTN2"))
 (segment (start 117 137.5) (end 117 122) (width 0.2) (layer "F.Cu") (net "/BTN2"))
 (segment (start 130.5 131) (end 127.5 134) (width 0.2) (layer "F.Cu") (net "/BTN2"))
 (segment (start 106.175 107.132) (end 106.175 107.175) (width 0.2) (layer "F.Cu") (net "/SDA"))
 (segment (start 108.5 107.132) (end 106.175 107.132) (width 0.2) (layer "F.Cu") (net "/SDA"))
 (segment (start 106.175 107.175) (end 106.5 107.5) (width 0.2) (layer "F.Cu") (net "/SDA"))
 (segment (start 121.445 126.33) (end 121.445 126.445) (width 0.2) (layer "F.Cu") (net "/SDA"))
 (segment (start 104 107.132) (end 106.175 107.132) (width 0.2) (layer "F.Cu") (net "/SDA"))
 (segment (start 121.445 126.445) (end 121.5 126.5) (width 0.2) (layer "F.Cu") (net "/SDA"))
 (segment (start 119.5 126.33) (end 121.445 126.33) (width 0.2) (layer "F.Cu") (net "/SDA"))
 (via (at 119.5 126.33) (size 0.6) (drill 0.3) (layers "F.Cu" "B.Cu") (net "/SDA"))
 (via (at 104 107.132) (size 0.6) (drill 0.3) (layers "F.Cu" "B.Cu") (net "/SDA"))
 (via (at 108.5 107.132) (size 0.6) (drill 0.3) (layers "F.Cu" "B.Cu") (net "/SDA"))
 (segment (start 116.5 126) (end 117 126.5) (width 0.2) (layer "B.Cu") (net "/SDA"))
 (segment (start 107.5 91.5) (end 119.5 91.5) (width 0.2) (layer "B.Cu") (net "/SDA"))
 (segment (start 111.5 108) (end 111.5 118) (width 0.2) (layer "B.Cu") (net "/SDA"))
 (segment (start 101.368 107.132) (end 100.5 108) (width 0.2) (layer "B.Cu") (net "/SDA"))
 (segment (start 111 107.5) (end 111.5 108) (width 0.2) (layer "B.Cu") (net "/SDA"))
 (segment (start 151.5 83.5) (end 145.5 83.5) (width 0.2) (layer "B.Cu") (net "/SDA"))
 (segment (start 119.33 126.5) (end 119.5 126.33) (width 0.2) (layer "B.Cu") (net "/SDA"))
 (segment (start 106.5 92.5) (end 107.5 91.5) (width 0.2) (layer "B.Cu") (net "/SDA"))
 (segment (start 111.5 118) (end 116 122.5) (width 0.2) (layer "B.Cu") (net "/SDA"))
 (segment (start 151.5 82.5) (end 151.5 83.5) (width 0.2) (layer "B.Cu") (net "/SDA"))
 (segment (start 147 78) (end 151.5 82.5) (width 0.2) (layer "B.Cu") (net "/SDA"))
 (segment (start 143.5 85.5) (end 143.5 91.08) (width 0.2) (layer "B.Cu") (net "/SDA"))
 (segment (start 147 75) (end 147 78) (width 0.2) (layer "B.Cu") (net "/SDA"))
 (segment (start 119.5 91.5) (end 123.5 87.5) (width 0.2) (layer "B.Cu") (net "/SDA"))
 (segment (start 143.5 91.08) (end 142.58 92) (width 0.2) (layer "B.Cu") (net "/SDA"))
 (segment (start 104 107.132) (end 101.368 107.132) (width 0.2) (layer "B.Cu") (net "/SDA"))
 (segment (start 116 126) (end 116.5 126) (width 0.2) (layer "B.Cu") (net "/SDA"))
 (segment (start 100.5 94) (end 102 92.5) (width 0.2) (layer "B.Cu") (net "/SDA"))
 (segment (start 116 122.5) (end 116 126) (width 0.2) (layer "B.Cu") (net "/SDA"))
 (segment (start 129 75) (end 147 75) (width 0.2) (layer "B.Cu") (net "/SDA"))
 (segment (start 123.5 87.5) (end 123.5 80.5) (width 0.2) (layer "B.Cu") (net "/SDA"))
 (segment (start 100.5 108) (end 100.5 94) (width 0.2) (layer "B.Cu") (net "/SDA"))
 (segment (start 123.5 80.5) (end 129 75) (width 0.2) (layer "B.Cu") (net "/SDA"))
 (segment (start 108.868 107.5) (end 111 107.5) (width 0.2) (layer "B.Cu") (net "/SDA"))
 (segment (start 117 126.5) (end 119.33 126.5) (width 0.2) (layer "B.Cu") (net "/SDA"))
 (segment (start 108.5 107.132) (end 108.868 107.5) (width 0.2) (layer "B.Cu") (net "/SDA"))
 (segment (start 102 92.5) (end 106.5 92.5) (width 0.2) (layer "B.Cu") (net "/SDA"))
 (segment (start 145.5 83.5) (end 143.5 85.5) (width 0.2) (layer "B.Cu") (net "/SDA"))
 (segment (start 108.672 109.672) (end 106.175 109.672) (width 0.2) (layer "F.Cu") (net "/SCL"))
 (segment (start 109 110) (end 108.672 109.672) (width 0.2) (layer "F.Cu") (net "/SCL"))
 (segment (start 124.755 125.755) (end 124.755 123.79) (width 0.2) (layer "F.Cu") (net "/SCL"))
 (segment (start 109.5 111.5) (end 109.5 110) (width 0.2) (layer "F.Cu") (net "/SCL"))
 (segment (start 127 124) (end 126.5 124) (width 0.2) (layer "F.Cu") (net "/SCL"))
 (segment (start 109.5 110) (end 109 110) (width 0.2) (layer "F.Cu") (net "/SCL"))
 (segment (start 126.5 124) (end 126.29 123.79) (width 0.2) (layer "F.Cu") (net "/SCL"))
 (segment (start 125 126) (end 124.755 125.755) (width 0.2) (layer "F.Cu") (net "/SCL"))
 (segment (start 126.29 123.79) (end 124.755 123.79) (width 0.2) (layer "F.Cu") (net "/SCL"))
 (via (at 109.5 111.5) (size 0.6) (drill 0.3) (layers "F.Cu" "B.Cu") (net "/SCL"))
 (via (at 127 124) (size 0.6) (drill 0.3) (layers "F.Cu" "B.Cu") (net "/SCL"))
 (via (at 125 126) (size 0.6) (drill 0.3) (layers "F.Cu" "B.Cu") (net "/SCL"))
 (segment (start 135 95.5) (end 139.5 95.5) (width 0.2) (layer "B.Cu") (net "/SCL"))
 (segment (start 109.5 113) (end 109.5 111.5) (width 0.2) (layer "B.Cu") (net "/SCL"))
 (segment (start 124.755 125.755) (end 125 126) (width 0.2) (layer "B.Cu") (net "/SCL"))
 (segment (start 122.5 128.5) (end 125 126) (width 0.2) (layer "B.Cu") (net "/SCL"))
 (segment (start 106.175 117.175) (end 106.175 116.325) (width 0.2) (layer "B.Cu") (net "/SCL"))
 (segment (start 140.04 94.96) (end 140.04 92) (width 0.2) (layer "B.Cu") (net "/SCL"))
 (segment (start 115.5 128.5) (end 122.5 128.5) (width 0.2) (layer "B.Cu") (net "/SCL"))
 (segment (start 106.175 116.325) (end 109.5 113) (width 0.2) (layer "B.Cu") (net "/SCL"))
 (segment (start 135 116.5) (end 135 95.5) (width 0.2) (layer "B.Cu") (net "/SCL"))
 (segment (start 127.5 124) (end 127 124) (width 0.2) (layer "B.Cu") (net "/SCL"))
 (segment (start 139.5 95.5) (end 140.04 94.96) (width 0.2) (layer "B.Cu") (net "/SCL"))
 (segment (start 135 116.5) (end 127.5 124) (width 0.2) (layer "B.Cu") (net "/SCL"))
 (segment (start 106.175 117.175) (end 115.5 126.5) (width 0.2) (layer "B.Cu") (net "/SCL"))
 (segment (start 115.5 126.5) (end 115.5 128.5) (width 0.2) (layer "B.Cu") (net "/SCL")))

